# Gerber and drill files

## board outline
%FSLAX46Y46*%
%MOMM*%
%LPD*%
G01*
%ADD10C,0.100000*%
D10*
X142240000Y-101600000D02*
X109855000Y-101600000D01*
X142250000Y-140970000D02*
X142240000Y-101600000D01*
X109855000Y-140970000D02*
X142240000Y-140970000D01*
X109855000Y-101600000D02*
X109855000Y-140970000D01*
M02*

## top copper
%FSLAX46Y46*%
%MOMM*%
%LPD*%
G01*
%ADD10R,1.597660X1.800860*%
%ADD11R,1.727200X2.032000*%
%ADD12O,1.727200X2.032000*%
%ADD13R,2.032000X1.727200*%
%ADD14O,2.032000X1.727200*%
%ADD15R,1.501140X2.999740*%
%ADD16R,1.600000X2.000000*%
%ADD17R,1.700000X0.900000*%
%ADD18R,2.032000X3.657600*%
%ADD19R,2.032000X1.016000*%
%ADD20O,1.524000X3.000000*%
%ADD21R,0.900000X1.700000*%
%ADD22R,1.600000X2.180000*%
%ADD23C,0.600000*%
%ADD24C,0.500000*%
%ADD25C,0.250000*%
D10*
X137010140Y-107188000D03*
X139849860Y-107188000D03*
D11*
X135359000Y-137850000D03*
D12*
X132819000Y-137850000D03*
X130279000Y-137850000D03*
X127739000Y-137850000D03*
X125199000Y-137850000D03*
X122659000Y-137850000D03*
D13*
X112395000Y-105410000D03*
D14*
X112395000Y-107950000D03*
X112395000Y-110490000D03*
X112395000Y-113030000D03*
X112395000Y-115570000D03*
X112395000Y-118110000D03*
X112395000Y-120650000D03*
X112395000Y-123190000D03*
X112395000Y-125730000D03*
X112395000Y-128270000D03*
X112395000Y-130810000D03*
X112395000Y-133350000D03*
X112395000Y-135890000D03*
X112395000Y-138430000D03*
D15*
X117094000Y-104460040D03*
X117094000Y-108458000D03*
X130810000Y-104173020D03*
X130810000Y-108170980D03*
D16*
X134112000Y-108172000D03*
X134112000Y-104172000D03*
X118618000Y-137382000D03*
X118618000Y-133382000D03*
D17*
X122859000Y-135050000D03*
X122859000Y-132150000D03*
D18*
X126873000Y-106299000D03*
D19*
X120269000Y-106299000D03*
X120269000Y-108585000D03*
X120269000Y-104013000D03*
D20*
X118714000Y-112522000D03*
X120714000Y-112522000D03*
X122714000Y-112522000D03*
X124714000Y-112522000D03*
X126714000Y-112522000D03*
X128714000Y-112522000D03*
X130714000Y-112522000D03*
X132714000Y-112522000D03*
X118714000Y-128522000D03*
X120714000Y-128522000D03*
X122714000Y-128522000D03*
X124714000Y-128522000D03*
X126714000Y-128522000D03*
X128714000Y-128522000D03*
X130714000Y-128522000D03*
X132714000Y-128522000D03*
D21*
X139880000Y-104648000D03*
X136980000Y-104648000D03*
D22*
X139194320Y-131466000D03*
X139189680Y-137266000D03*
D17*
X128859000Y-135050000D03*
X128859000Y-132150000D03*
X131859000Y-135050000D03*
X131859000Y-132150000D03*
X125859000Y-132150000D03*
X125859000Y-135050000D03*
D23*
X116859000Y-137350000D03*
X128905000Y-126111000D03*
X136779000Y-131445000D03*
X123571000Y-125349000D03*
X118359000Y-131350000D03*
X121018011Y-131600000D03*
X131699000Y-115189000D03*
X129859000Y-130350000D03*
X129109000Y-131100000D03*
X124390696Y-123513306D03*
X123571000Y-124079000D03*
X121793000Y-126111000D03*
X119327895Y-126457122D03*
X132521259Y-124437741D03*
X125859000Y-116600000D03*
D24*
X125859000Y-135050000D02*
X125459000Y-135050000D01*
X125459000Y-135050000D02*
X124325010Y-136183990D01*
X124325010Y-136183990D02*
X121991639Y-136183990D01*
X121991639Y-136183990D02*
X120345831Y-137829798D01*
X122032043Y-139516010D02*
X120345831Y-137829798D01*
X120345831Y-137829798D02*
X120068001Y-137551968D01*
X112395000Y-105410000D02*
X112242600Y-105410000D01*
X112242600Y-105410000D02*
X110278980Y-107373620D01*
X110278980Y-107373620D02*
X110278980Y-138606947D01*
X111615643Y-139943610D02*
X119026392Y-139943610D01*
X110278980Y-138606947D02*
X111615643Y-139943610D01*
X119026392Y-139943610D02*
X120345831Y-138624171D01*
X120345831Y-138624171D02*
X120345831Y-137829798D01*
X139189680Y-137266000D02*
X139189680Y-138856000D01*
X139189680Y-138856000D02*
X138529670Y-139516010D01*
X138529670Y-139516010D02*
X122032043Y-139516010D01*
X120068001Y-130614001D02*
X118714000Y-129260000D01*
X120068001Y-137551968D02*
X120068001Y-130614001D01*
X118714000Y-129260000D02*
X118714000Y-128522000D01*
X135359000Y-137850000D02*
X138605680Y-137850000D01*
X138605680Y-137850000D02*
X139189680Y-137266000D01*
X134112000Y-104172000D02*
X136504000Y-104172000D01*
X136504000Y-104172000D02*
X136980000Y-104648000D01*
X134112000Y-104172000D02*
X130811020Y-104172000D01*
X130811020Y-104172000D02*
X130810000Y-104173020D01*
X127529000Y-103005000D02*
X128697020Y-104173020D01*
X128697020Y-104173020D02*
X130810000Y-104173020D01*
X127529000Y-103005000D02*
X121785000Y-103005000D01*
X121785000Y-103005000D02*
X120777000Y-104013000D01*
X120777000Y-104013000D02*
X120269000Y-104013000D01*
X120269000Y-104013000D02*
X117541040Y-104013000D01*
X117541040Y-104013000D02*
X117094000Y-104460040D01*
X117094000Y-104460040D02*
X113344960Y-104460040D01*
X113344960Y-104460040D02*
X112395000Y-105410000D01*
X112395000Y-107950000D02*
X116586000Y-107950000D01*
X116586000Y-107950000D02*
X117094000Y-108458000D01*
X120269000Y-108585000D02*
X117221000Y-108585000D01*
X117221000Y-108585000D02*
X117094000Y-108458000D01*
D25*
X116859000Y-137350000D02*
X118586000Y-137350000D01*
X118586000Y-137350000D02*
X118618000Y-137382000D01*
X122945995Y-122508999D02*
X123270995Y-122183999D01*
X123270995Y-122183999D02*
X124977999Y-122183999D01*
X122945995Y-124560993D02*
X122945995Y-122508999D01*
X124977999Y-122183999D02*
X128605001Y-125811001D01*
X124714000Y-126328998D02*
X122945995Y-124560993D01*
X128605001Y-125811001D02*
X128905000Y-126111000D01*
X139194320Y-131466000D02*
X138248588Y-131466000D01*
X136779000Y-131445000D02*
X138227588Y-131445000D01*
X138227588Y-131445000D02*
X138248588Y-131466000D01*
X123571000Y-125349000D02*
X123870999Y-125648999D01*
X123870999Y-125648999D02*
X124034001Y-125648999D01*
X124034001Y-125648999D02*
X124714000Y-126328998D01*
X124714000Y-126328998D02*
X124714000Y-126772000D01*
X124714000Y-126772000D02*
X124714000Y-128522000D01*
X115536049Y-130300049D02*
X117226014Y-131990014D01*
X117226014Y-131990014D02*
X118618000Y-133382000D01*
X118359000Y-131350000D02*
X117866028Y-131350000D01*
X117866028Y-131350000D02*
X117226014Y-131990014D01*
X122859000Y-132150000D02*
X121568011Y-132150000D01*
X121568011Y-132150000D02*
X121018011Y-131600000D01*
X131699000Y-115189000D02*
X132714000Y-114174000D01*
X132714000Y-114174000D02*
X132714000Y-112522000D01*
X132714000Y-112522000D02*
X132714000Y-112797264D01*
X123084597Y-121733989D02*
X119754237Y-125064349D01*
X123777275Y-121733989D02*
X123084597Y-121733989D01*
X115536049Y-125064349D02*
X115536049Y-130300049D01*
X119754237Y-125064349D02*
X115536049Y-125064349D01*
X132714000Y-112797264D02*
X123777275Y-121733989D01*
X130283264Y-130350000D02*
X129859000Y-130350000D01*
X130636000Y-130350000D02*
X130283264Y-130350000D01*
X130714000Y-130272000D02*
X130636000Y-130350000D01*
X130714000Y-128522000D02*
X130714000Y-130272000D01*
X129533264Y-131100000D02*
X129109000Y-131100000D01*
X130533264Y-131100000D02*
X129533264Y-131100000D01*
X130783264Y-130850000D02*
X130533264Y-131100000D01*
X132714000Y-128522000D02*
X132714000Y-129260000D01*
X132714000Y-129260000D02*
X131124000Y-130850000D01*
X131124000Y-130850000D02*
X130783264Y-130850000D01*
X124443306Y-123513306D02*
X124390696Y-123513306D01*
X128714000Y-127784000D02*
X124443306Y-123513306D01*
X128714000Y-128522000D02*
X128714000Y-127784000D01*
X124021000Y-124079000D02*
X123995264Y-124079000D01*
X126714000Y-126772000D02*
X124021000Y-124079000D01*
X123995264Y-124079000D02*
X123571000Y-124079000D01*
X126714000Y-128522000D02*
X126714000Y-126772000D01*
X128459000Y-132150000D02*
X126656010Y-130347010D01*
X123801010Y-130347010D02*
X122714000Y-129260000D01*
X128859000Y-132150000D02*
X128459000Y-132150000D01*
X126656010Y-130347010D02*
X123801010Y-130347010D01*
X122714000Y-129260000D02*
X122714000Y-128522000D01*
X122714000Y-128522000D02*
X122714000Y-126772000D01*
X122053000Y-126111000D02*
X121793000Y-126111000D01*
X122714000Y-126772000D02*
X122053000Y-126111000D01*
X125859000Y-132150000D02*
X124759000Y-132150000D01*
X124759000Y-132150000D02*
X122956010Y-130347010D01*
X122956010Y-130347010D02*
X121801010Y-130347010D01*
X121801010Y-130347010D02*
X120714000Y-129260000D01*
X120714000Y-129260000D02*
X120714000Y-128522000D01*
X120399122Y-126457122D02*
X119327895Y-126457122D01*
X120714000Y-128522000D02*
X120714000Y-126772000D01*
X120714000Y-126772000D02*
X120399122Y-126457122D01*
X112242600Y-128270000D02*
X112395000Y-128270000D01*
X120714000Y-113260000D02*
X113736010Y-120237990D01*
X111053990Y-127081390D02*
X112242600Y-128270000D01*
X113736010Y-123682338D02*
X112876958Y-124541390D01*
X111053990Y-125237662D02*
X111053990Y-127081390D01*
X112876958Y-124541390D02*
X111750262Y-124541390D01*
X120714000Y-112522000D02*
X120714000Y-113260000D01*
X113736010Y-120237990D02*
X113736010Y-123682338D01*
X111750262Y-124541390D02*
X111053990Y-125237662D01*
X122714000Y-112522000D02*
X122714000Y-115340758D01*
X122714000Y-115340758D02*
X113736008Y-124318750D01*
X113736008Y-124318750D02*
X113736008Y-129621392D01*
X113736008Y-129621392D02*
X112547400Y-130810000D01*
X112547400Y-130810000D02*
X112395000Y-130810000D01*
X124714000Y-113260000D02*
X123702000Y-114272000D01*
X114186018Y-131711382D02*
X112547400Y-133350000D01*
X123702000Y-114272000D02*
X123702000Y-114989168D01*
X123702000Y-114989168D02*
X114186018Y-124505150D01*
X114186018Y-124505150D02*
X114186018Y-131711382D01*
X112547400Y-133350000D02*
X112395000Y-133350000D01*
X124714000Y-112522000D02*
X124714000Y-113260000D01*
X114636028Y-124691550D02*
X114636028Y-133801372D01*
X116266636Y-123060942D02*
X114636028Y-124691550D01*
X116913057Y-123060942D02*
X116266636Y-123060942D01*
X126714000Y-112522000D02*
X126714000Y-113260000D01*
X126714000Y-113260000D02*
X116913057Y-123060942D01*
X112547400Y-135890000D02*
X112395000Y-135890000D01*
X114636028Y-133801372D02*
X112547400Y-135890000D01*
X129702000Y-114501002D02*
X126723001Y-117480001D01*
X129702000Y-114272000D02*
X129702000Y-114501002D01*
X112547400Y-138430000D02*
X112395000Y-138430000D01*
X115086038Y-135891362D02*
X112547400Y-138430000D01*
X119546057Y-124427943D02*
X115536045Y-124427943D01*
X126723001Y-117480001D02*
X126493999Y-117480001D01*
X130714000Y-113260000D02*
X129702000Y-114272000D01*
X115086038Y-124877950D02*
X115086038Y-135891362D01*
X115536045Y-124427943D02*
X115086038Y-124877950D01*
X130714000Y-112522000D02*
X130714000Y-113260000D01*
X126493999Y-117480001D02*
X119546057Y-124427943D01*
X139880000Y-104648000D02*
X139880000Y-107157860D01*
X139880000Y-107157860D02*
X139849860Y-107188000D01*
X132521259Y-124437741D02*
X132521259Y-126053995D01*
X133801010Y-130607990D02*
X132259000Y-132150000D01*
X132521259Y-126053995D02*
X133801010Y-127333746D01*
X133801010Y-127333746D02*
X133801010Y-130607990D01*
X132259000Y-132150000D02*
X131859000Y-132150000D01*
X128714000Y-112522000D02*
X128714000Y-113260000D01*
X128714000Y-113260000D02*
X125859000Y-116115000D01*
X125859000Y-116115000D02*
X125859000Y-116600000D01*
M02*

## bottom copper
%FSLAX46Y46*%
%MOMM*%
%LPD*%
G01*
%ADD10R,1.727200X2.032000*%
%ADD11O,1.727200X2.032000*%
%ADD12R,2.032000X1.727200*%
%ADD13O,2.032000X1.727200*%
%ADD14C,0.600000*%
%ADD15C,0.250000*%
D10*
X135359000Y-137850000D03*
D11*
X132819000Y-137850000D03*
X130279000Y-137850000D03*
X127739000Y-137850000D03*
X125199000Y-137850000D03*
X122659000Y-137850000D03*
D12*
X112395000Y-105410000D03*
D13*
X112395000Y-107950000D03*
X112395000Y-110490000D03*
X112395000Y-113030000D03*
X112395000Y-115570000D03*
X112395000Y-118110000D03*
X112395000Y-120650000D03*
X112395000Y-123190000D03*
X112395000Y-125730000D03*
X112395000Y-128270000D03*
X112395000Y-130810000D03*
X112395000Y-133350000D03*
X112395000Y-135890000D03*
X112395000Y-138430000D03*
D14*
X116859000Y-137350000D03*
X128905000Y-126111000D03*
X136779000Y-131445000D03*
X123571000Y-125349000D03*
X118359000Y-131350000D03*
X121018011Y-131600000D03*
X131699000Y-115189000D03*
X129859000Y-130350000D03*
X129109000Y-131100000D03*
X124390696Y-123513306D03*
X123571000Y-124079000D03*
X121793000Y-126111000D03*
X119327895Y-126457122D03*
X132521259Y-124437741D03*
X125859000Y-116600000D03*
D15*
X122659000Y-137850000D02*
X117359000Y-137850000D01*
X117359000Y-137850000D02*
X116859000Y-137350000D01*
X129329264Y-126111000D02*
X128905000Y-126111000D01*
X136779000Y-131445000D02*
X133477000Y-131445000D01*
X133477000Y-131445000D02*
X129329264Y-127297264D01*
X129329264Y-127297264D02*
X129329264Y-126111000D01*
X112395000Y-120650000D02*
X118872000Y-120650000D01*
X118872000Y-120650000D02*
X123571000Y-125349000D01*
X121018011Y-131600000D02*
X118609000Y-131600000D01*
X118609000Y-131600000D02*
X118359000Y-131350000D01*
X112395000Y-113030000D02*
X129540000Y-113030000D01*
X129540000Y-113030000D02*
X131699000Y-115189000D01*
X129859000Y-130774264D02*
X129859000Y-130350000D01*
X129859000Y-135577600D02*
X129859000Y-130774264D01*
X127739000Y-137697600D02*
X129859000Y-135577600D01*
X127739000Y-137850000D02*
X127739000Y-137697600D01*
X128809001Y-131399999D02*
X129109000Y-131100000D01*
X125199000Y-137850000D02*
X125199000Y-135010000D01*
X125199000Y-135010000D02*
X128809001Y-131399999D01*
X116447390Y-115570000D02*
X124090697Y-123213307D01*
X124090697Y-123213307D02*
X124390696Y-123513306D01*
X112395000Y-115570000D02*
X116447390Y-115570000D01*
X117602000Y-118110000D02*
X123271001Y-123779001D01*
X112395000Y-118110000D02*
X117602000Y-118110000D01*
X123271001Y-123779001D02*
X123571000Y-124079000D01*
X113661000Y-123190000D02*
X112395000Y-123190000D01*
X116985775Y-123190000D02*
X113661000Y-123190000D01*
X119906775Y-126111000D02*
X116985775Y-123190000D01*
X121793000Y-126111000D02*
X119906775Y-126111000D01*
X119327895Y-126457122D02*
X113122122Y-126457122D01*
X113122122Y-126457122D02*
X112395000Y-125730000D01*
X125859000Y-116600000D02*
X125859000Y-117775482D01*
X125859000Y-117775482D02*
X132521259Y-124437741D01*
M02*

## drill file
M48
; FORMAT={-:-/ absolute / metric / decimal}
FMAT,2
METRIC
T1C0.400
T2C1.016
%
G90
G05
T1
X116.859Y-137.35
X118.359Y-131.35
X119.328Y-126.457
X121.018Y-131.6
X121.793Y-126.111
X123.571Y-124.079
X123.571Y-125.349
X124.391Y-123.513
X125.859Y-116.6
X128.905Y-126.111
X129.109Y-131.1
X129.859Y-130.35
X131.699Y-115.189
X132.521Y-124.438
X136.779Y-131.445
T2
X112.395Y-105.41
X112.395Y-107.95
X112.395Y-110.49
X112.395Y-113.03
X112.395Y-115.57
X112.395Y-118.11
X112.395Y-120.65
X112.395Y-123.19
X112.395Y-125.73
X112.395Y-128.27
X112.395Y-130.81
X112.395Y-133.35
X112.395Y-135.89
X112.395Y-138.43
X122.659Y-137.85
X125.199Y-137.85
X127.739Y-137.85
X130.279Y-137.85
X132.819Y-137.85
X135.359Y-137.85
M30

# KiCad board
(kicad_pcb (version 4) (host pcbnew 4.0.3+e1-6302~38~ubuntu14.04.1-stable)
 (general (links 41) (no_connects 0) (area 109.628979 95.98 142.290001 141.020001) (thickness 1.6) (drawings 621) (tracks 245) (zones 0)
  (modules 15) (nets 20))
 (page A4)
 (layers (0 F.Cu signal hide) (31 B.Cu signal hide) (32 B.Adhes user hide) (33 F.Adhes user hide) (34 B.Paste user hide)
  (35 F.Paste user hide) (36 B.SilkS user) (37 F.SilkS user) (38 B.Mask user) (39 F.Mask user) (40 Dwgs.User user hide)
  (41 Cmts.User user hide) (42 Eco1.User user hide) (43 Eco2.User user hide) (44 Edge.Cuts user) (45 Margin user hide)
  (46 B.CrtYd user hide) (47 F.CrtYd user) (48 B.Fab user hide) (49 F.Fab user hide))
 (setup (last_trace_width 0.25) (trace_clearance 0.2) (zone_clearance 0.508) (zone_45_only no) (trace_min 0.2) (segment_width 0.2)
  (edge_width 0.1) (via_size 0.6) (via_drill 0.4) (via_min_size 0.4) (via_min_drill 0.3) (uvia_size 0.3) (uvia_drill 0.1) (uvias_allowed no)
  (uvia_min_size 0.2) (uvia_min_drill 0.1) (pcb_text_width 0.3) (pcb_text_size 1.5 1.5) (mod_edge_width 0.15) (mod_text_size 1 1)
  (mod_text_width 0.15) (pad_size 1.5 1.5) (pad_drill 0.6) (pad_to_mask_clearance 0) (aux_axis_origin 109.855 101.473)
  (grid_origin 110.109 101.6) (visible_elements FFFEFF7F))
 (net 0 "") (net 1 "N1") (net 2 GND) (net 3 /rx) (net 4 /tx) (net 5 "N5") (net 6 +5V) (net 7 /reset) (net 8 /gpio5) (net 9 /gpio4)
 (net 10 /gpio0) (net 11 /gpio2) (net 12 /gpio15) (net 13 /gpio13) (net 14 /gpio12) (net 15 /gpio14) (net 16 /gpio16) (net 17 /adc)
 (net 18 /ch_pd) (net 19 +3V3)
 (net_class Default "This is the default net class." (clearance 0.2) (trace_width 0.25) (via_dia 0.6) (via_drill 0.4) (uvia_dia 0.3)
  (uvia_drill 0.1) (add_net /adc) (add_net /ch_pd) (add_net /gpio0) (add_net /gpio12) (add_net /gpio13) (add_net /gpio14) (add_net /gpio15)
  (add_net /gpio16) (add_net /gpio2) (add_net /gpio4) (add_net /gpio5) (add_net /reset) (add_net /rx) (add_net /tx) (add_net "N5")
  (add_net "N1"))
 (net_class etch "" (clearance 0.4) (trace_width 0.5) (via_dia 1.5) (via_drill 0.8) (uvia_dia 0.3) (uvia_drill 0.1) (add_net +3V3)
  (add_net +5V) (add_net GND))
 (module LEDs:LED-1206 (layer F.Cu) (at 138.43 107.188 180)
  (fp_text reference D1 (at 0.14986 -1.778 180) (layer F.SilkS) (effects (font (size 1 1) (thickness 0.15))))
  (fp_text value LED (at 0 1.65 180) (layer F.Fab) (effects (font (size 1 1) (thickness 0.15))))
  (pad 2 smd rect (at 1.41986 0) (size 1.59766 1.80086) (layers F.Cu F.Paste F.Mask))
  (pad 1 smd rect (at -1.41986 0) (size 1.59766 1.80086) (layers F.Cu F.Paste F.Mask) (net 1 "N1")))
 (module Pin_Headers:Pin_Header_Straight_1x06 (layer F.Cu) (at 135.359 137.85 270)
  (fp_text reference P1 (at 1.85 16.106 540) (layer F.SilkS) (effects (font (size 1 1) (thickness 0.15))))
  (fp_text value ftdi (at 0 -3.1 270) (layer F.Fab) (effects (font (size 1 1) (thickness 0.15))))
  (pad 1 thru_hole rect (at 0 0 270) (size 2.032 1.7272) (drill 1.016) (layers *.Cu *.Mask F.SilkS) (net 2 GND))
  (pad 2 thru_hole oval (at 0 2.54 270) (size 2.032 1.7272) (drill 1.016) (layers *.Cu *.Mask F.SilkS))
  (pad 3 thru_hole oval (at 0 5.08 270) (size 2.032 1.7272) (drill 1.016) (layers *.Cu *.Mask F.SilkS))
  (pad 4 thru_hole oval (at 0 7.62 270) (size 2.032 1.7272) (drill 1.016) (layers *.Cu *.Mask F.SilkS) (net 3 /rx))
  (pad 5 thru_hole oval (at 0 10.16 270) (size 2.032 1.7272) (drill 1.016) (layers *.Cu *.Mask F.SilkS) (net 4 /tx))
  (pad 6 thru_hole oval (at 0 12.7 270) (size 2.032 1.7272) (drill 1.016) (layers *.Cu *.Mask F.SilkS) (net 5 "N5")))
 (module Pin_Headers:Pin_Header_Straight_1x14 (layer B.Cu) (at 112.395 105.41 180)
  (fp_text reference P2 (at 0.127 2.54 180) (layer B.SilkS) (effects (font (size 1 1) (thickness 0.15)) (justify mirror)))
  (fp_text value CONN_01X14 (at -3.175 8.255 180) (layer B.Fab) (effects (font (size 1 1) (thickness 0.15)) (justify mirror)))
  (pad 1 thru_hole rect (at 0 0 180) (size 2.032 1.7272) (drill 1.016) (layers *.Cu *.Mask B.SilkS) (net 2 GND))
  (pad 2 thru_hole oval (at 0 -2.54 180) (size 2.032 1.7272) (drill 1.016) (layers *.Cu *.Mask B.SilkS) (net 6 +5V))
  (pad 3 thru_hole oval (at 0 -5.08 180) (size 2.032 1.7272) (drill 1.016) (layers *.Cu *.Mask B.SilkS))
  (pad 4 thru_hole oval (at 0 -7.62 180) (size 2.032 1.7272) (drill 1.016) (layers *.Cu *.Mask B.SilkS) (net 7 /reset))
  (pad 5 thru_hole oval (at 0 -10.16 180) (size 2.032 1.7272) (drill 1.016) (layers *.Cu *.Mask B.SilkS) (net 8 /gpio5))
  (pad 6 thru_hole oval (at 0 -12.7 180) (size 2.032 1.7272) (drill 1.016) (layers *.Cu *.Mask B.SilkS) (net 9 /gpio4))
  (pad 7 thru_hole oval (at 0 -15.24 180) (size 2.032 1.7272) (drill 1.016) (layers *.Cu *.Mask B.SilkS) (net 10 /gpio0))
  (pad 8 thru_hole oval (at 0 -17.78 180) (size 2.032 1.7272) (drill 1.016) (layers *.Cu *.Mask B.SilkS) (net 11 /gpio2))
  (pad 9 thru_hole oval (at 0 -20.32 180) (size 2.032 1.7272) (drill 1.016) (layers *.Cu *.Mask B.SilkS) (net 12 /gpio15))
  (pad 10 thru_hole oval (at 0 -22.86 180) (size 2.032 1.7272) (drill 1.016) (layers *.Cu *.Mask B.SilkS) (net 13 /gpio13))
  (pad 11 thru_hole oval (at 0 -25.4 180) (size 2.032 1.7272) (drill 1.016) (layers *.Cu *.Mask B.SilkS) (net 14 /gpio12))
  (pad 12 thru_hole oval (at 0 -27.94 180) (size 2.032 1.7272) (drill 1.016) (layers *.Cu *.Mask B.SilkS) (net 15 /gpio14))
  (pad 13 thru_hole oval (at 0 -30.48 180) (size 2.032 1.7272) (drill 1.016) (layers *.Cu *.Mask B.SilkS) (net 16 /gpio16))
  (pad 14 thru_hole oval (at 0 -33.02 180) (size 2.032 1.7272) (drill 1.016) (layers *.Cu *.Mask B.SilkS) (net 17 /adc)))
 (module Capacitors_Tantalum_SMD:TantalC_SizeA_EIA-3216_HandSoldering (layer F.Cu) (at 117.094 106.45902 90)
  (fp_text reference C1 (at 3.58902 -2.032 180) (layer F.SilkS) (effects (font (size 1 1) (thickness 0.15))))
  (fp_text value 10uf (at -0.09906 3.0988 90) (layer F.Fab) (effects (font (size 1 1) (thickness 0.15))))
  (pad 2 smd rect (at 1.99898 0 90) (size 2.99974 1.50114) (layers F.Cu F.Paste F.Mask) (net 2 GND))
  (pad 1 smd rect (at -1.99898 0 90) (size 2.99974 1.50114) (layers F.Cu F.Paste F.Mask) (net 6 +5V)))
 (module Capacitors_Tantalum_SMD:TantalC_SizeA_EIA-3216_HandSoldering (layer F.Cu) (at 130.81 106.172 90)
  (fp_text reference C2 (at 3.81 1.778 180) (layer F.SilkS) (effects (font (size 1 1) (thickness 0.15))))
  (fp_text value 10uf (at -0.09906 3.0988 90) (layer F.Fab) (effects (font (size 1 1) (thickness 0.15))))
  (pad 2 smd rect (at 1.99898 0 90) (size 2.99974 1.50114) (layers F.Cu F.Paste F.Mask) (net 2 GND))
  (pad 1 smd rect (at -1.99898 0 90) (size 2.99974 1.50114) (layers F.Cu F.Paste F.Mask)))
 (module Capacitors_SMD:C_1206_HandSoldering (layer F.Cu) (at 134.112 106.172 90)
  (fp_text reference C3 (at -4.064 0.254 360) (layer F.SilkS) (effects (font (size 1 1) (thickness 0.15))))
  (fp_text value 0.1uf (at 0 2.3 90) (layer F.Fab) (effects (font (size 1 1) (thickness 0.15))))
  (pad 1 smd rect (at -2 0 90) (size 2 1.6) (layers F.Cu F.Paste F.Mask))
  (pad 2 smd rect (at 2 0 90) (size 2 1.6) (layers F.Cu F.Paste F.Mask) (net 2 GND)))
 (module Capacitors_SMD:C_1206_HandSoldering (layer F.Cu) (at 118.618 135.382 90)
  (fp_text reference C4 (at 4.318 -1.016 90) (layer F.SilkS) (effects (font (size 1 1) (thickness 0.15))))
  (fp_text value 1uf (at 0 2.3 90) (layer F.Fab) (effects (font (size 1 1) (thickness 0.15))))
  (pad 1 smd rect (at -2 0 90) (size 2 1.6) (layers F.Cu F.Paste F.Mask) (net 5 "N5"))
  (pad 2 smd rect (at 2 0 90) (size 2 1.6) (layers F.Cu F.Paste F.Mask) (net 7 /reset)))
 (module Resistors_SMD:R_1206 (layer F.Cu) (at 122.859 133.6 90)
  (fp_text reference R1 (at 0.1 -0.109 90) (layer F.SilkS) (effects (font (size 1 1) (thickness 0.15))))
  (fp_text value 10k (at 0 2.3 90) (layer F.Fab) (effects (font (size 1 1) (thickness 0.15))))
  (pad 1 smd rect (at -1.45 0 90) (size 0.9 1.7) (layers F.Cu F.Paste F.Mask))
  (pad 2 smd rect (at 1.45 0 90) (size 0.9 1.7) (layers F.Cu F.Paste F.Mask) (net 7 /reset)))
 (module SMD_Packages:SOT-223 (layer F.Cu) (at 123.571 106.299 270)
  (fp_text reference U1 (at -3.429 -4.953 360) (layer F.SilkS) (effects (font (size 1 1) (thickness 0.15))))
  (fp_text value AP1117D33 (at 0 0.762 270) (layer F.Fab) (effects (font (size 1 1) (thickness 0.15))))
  (pad 4 smd rect (at 0 -3.302 270) (size 3.6576 2.032) (layers F.Cu F.Paste F.Mask))
  (pad 2 smd rect (at 0 3.302 270) (size 1.016 2.032) (layers F.Cu F.Paste F.Mask))
  (pad 3 smd rect (at 2.286 3.302 270) (size 1.016 2.032) (layers F.Cu F.Paste F.Mask) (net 6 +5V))
  (pad 1 smd rect (at -2.286 3.302 270) (size 1.016 2.032) (layers F.Cu F.Paste F.Mask) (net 2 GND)))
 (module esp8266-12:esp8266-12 (layer F.Cu) (at 118.714 112.622)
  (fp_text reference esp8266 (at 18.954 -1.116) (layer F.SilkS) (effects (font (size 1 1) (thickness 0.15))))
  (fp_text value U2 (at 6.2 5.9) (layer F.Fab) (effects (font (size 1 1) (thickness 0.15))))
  (pad 8 smd oval (at 0 -0.1) (size 1.524 3) (layers F.Cu F.Paste F.Mask))
  (pad 7 smd oval (at 2 -0.1) (size 1.524 3) (layers F.Cu F.Paste F.Mask) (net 13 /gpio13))
  (pad 6 smd oval (at 4 -0.1) (size 1.524 3) (layers F.Cu F.Paste F.Mask) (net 14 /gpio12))
  (pad 5 smd oval (at 6 -0.1) (size 1.524 3) (layers F.Cu F.Paste F.Mask) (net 15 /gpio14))
  (pad 4 smd oval (at 8 -0.1) (size 1.524 3) (layers F.Cu F.Paste F.Mask) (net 16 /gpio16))
  (pad 3 smd oval (at 10 -0.1) (size 1.524 3) (layers F.Cu F.Paste F.Mask) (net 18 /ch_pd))
  (pad 2 smd oval (at 12 -0.1) (size 1.524 3) (layers F.Cu F.Paste F.Mask) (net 17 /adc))
  (pad 1 smd oval (at 14 -0.1) (size 1.524 3) (layers F.Cu F.Paste F.Mask) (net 7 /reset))
  (pad 9 smd oval (at 0 15.9) (size 1.524 3) (layers F.Cu F.Paste F.Mask) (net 2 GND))
  (pad 10 smd oval (at 2 15.9) (size 1.524 3) (layers F.Cu F.Paste F.Mask) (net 12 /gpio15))
  (pad 11 smd oval (at 4 15.9) (size 1.524 3) (layers F.Cu F.Paste F.Mask) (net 11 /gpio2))
  (pad 12 smd oval (at 6 15.9) (size 1.524 3) (layers F.Cu F.Paste F.Mask) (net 10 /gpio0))
  (pad 13 smd oval (at 8 15.9) (size 1.524 3) (layers F.Cu F.Paste F.Mask) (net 9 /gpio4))
  (pad 14 smd oval (at 10 15.9) (size 1.524 3) (layers F.Cu F.Paste F.Mask) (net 8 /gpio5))
  (pad 15 smd oval (at 12 15.9) (size 1.524 3) (layers F.Cu F.Paste F.Mask) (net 3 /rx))
  (pad 16 smd oval (at 14 15.9) (size 1.524 3) (layers F.Cu F.Paste F.Mask) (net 4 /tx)))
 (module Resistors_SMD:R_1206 (layer F.Cu) (at 138.43 104.648 180)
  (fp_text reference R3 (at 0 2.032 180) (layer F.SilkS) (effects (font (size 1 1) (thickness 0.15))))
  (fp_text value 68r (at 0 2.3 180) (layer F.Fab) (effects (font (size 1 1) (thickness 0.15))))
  (pad 1 smd rect (at -1.45 0 180) (size 0.9 1.7) (layers F.Cu F.Paste F.Mask) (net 1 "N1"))
  (pad 2 smd rect (at 1.45 0 180) (size 0.9 1.7) (layers F.Cu F.Paste F.Mask) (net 2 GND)))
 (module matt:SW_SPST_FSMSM (layer F.Cu) (at 139.192 134.366 270)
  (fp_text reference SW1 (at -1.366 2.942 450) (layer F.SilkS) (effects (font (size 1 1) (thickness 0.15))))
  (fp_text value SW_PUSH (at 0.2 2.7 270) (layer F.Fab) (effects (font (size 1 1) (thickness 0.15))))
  (pad 1 smd rect (at -2.9 -0.00232 270) (size 2.18 1.6) (layers F.Cu F.Paste F.Mask) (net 10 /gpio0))
  (pad 2 smd rect (at 2.9 0.00232 270) (size 2.18 1.6) (layers F.Cu F.Paste F.Mask) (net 2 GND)))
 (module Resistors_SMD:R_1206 (layer F.Cu) (at 128.859 133.6 90)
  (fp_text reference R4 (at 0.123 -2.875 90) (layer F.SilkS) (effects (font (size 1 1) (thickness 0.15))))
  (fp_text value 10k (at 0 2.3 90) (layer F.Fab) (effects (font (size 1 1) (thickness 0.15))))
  (pad 1 smd rect (at -1.45 0 90) (size 0.9 1.7) (layers F.Cu F.Paste F.Mask))
  (pad 2 smd rect (at 1.45 0 90) (size 0.9 1.7) (layers F.Cu F.Paste F.Mask) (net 11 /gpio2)))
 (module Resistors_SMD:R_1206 (layer F.Cu) (at 131.859 133.6 90)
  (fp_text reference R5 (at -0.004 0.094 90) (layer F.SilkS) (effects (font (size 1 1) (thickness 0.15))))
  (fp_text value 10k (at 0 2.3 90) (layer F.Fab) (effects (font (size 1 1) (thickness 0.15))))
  (pad 1 smd rect (at -1.45 0 90) (size 0.9 1.7) (layers F.Cu F.Paste F.Mask))
  (pad 2 smd rect (at 1.45 0 90) (size 0.9 1.7) (layers F.Cu F.Paste F.Mask) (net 18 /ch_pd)))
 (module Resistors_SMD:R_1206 (layer F.Cu) (at 125.859 133.6 270)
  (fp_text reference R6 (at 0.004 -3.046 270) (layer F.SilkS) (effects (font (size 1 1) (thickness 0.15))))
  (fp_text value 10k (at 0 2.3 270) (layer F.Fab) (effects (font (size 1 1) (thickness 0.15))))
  (pad 1 smd rect (at -1.45 0 270) (size 0.9 1.7) (layers F.Cu F.Paste F.Mask) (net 12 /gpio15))
  (pad 2 smd rect (at 1.45 0 270) (size 0.9 1.7) (layers F.Cu F.Paste F.Mask) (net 2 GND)))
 (gr_line (start 142.24 101.6) (end 109.855 101.6) (layer Edge.Cuts) (width 0.1))
 (gr_line (start 142.25 140.97) (end 142.24 101.6) (layer Edge.Cuts) (width 0.1))
 (gr_line (start 109.855 140.97) (end 142.24 140.97) (layer Edge.Cuts) (width 0.1))
 (gr_line (start 109.855 101.6) (end 109.855 140.97) (layer Edge.Cuts) (width 0.1))
 (segment (start 125.859 135.05) (end 125.459 135.05) (width 0.5) (layer F.Cu) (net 2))
 (segment (start 125.459 135.05) (end 124.32501 136.18399) (width 0.5) (layer F.Cu) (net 2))
 (segment (start 124.32501 136.18399) (end 121.991639 136.18399) (width 0.5) (layer F.Cu) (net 2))
 (segment (start 121.991639 136.18399) (end 120.345831 137.829798) (width 0.5) (layer F.Cu) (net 2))
 (segment (start 122.032043 139.51601) (end 120.345831 137.829798) (width 0.5) (layer F.Cu) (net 2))
 (segment (start 120.345831 137.829798) (end 120.068001 137.551968) (width 0.5) (layer F.Cu) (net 2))
 (segment (start 112.395 105.41) (end 112.2426 105.41) (width 0.5) (layer F.Cu) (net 2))
 (segment (start 112.2426 105.41) (end 110.27898 107.37362) (width 0.5) (layer F.Cu) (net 2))
 (segment (start 110.27898 107.37362) (end 110.27898 138.606947) (width 0.5) (layer F.Cu) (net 2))
 (segment (start 111.615643 139.94361) (end 119.026392 139.94361) (width 0.5) (layer F.Cu) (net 2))
 (segment (start 110.27898 138.606947) (end 111.615643 139.94361) (width 0.5) (layer F.Cu) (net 2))
 (segment (start 119.026392 139.94361) (end 120.345831 138.624171) (width 0.5) (layer F.Cu) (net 2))
 (segment (start 120.345831 138.624171) (end 120.345831 137.829798) (width 0.5) (layer F.Cu) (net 2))
 (segment (start 139.18968 137.266) (end 139.18968 138.856) (width 0.5) (layer F.Cu) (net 2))
 (segment (start 139.18968 138.856) (end 138.52967 139.51601) (width 0.5) (layer F.Cu) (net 2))
 (segment (start 138.52967 139.51601) (end 122.032043 139.51601) (width 0.5) (layer F.Cu) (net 2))
 (segment (start 120.068001 130.614001) (end 118.714 129.26) (width 0.5) (layer F.Cu) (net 2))
 (segment (start 120.068001 137.551968) (end 120.068001 130.614001) (width 0.5) (layer F.Cu) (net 2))
 (segment (start 118.714 129.26) (end 118.714 128.522) (width 0.5) (layer F.Cu) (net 2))
 (segment (start 135.359 137.85) (end 138.60568 137.85) (width 0.5) (layer F.Cu) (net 2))
 (segment (start 138.60568 137.85) (end 139.18968 137.266) (width 0.5) (layer F.Cu) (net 2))
 (segment (start 134.112 104.172) (end 136.504 104.172) (width 0.5) (layer F.Cu) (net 2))
 (segment (start 136.504 104.172) (end 136.98 104.648) (width 0.5) (layer F.Cu) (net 2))
 (segment (start 134.112 104.172) (end 130.81102 104.172) (width 0.5) (layer F.Cu) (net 2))
 (segment (start 130.81102 104.172) (end 130.81 104.17302) (width 0.5) (layer F.Cu) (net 2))
 (segment (start 127.529 103.005) (end 128.69702 104.17302) (width 0.5) (layer F.Cu) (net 2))
 (segment (start 128.69702 104.17302) (end 130.81 104.17302) (width 0.5) (layer F.Cu) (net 2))
 (segment (start 127.529 103.005) (end 121.785 103.005) (width 0.5) (layer F.Cu) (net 2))
 (segment (start 121.785 103.005) (end 120.777 104.013) (width 0.5) (layer F.Cu) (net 2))
 (segment (start 120.777 104.013) (end 120.269 104.013) (width 0.5) (layer F.Cu) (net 2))
 (segment (start 120.269 104.013) (end 117.54104 104.013) (width 0.5) (layer F.Cu) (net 2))
 (segment (start 117.54104 104.013) (end 117.094 104.46004) (width 0.5) (layer F.Cu) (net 2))
 (segment (start 117.094 104.46004) (end 113.34496 104.46004) (width 0.5) (layer F.Cu) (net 2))
 (segment (start 113.34496 104.46004) (end 112.395 105.41) (width 0.5) (layer F.Cu) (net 2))
 (segment (start 112.395 107.95) (end 116.586 107.95) (width 0.5) (layer F.Cu) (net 6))
 (segment (start 116.586 107.95) (end 117.094 108.458) (width 0.5) (layer F.Cu) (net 6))
 (segment (start 120.269 108.585) (end 117.221 108.585) (width 0.5) (layer F.Cu) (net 6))
 (segment (start 117.221 108.585) (end 117.094 108.458) (width 0.5) (layer F.Cu) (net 6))
 (segment (start 116.859 137.35) (end 118.586 137.35) (width 0.25) (layer F.Cu) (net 5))
 (segment (start 118.586 137.35) (end 118.618 137.382) (width 0.25) (layer F.Cu) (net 5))
 (segment (start 122.659 137.85) (end 117.359 137.85) (width 0.25) (layer B.Cu) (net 5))
 (segment (start 117.359 137.85) (end 116.859 137.35) (width 0.25) (layer B.Cu) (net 5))
 (segment (start 122.945995 122.508999) (end 123.270995 122.183999) (width 0.25) (layer F.Cu) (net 10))
 (segment (start 123.270995 122.183999) (end 124.977999 122.183999) (width 0.25) (layer F.Cu) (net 10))
 (segment (start 122.945995 124.560993) (end 122.945995 122.508999) (width 0.25) (layer F.Cu) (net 10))
 (segment (start 124.977999 122.183999) (end 128.605001 125.811001) (width 0.25) (layer F.Cu) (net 10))
 (segment (start 124.714 126.328998) (end 122.945995 124.560993) (width 0.25) (layer F.Cu) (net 10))
 (segment (start 128.605001 125.811001) (end 128.905 126.111) (width 0.25) (layer F.Cu) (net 10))
 (segment (start 129.329264 126.111) (end 128.905 126.111) (width 0.25) (layer B.Cu) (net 10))
 (segment (start 136.779 131.445) (end 133.477 131.445) (width 0.25) (layer B.Cu) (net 10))
 (segment (start 133.477 131.445) (end 129.329264 127.297264) (width 0.25) (layer B.Cu) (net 10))
 (segment (start 129.329264 127.297264) (end 129.329264 126.111) (width 0.25) (layer B.Cu) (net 10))
 (segment (start 139.19432 131.466) (end 138.248588 131.466) (width 0.25) (layer F.Cu) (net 10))
 (segment (start 136.779 131.445) (end 138.227588 131.445) (width 0.25) (layer F.Cu) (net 10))
 (segment (start 138.227588 131.445) (end 138.248588 131.466) (width 0.25) (layer F.Cu) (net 10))
 (segment (start 123.571 125.349) (end 123.870999 125.648999) (width 0.25) (layer F.Cu) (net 10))
 (segment (start 123.870999 125.648999) (end 124.034001 125.648999) (width 0.25) (layer F.Cu) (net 10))
 (segment (start 124.034001 125.648999) (end 124.714 126.328998) (width 0.25) (layer F.Cu) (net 10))
 (segment (start 112.395 120.65) (end 118.872 120.65) (width 0.25) (layer B.Cu) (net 10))
 (segment (start 118.872 120.65) (end 123.571 125.349) (width 0.25) (layer B.Cu) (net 10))
 (segment (start 124.714 126.328998) (end 124.714 126.772) (width 0.25) (layer F.Cu) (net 10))
 (segment (start 124.714 126.772) (end 124.714 128.522) (width 0.25) (layer F.Cu) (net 10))
 (segment (start 115.536049 130.300049) (end 117.226014 131.990014) (width 0.25) (layer F.Cu) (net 7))
 (segment (start 117.226014 131.990014) (end 118.618 133.382) (width 0.25) (layer F.Cu) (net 7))
 (segment (start 118.359 131.35) (end 117.866028 131.35) (width 0.25) (layer F.Cu) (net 7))
 (segment (start 117.866028 131.35) (end 117.226014 131.990014) (width 0.25) (layer F.Cu) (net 7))
 (segment (start 121.018011 131.6) (end 118.609 131.6) (width 0.25) (layer B.Cu) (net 7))
 (segment (start 118.609 131.6) (end 118.359 131.35) (width 0.25) (layer B.Cu) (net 7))
 (segment (start 122.859 132.15) (end 121.568011 132.15) (width 0.25) (layer F.Cu) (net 7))
 (segment (start 121.568011 132.15) (end 121.018011 131.6) (width 0.25) (layer F.Cu) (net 7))
 (segment (start 131.699 115.189) (end 132.714 114.174) (width 0.25) (layer F.Cu) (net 7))
 (segment (start 132.714 114.174) (end 132.714 112.522) (width 0.25) (layer F.Cu) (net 7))
 (segment (start 112.395 113.03) (end 129.54 113.03) (width 0.25) (layer B.Cu) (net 7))
 (segment (start 129.54 113.03) (end 131.699 115.189) (width 0.25) (layer B.Cu) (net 7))
 (segment (start 132.714 112.522) (end 132.714 112.797264) (width 0.25) (layer F.Cu) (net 7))
 (segment (start 123.084597 121.733989) (end 119.754237 125.064349) (width 0.25) (layer F.Cu) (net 7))
 (segment (start 123.777275 121.733989) (end 123.084597 121.733989) (width 0.25) (layer F.Cu) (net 7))
 (segment (start 115.536049 125.064349) (end 115.536049 130.300049) (width 0.25) (layer F.Cu) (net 7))
 (segment (start 119.754237 125.064349) (end 115.536049 125.064349) (width 0.25) (layer F.Cu) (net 7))
 (segment (start 132.714 112.797264) (end 123.777275 121.733989) (width 0.25) (layer F.Cu) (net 7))
 (segment (start 129.859 130.774264) (end 129.859 130.35) (width 0.25) (layer B.Cu) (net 3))
 (segment (start 129.859 135.5776) (end 129.859 130.774264) (width 0.25) (layer B.Cu) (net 3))
 (segment (start 127.739 137.6976) (end 129.859 135.5776) (width 0.25) (layer B.Cu) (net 3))
 (segment (start 130.283264 130.35) (end 129.859 130.35) (width 0.25) (layer F.Cu) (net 3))
 (segment (start 130.636 130.35) (end 130.283264 130.35) (width 0.25) (layer F.Cu) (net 3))
 (segment (start 127.739 137.85) (end 127.739 137.6976) (width 0.25) (layer B.Cu) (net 3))
 (segment (start 130.714 130.272) (end 130.636 130.35) (width 0.25) (layer F.Cu) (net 3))
 (segment (start 130.714 128.522) (end 130.714 130.272) (width 0.25) (layer F.Cu) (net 3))
 (segment (start 128.809001 131.399999) (end 129.109 131.1) (width 0.25) (layer B.Cu) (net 4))
 (segment (start 125.199 137.85) (end 125.199 135.01) (width 0.25) (layer B.Cu) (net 4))
 (segment (start 125.199 135.01) (end 128.809001 131.399999) (width 0.25) (layer B.Cu) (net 4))
 (segment (start 129.533264 131.1) (end 129.109 131.1) (width 0.25) (layer F.Cu) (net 4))
 (segment (start 130.533264 131.1) (end 129.533264 131.1) (width 0.25) (layer F.Cu) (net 4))
 (segment (start 130.783264 130.85) (end 130.533264 131.1) (width 0.25) (layer F.Cu) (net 4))
 (segment (start 132.714 128.522) (end 132.714 129.26) (width 0.25) (layer F.Cu) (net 4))
 (segment (start 132.714 129.26) (end 131.124 130.85) (width 0.25) (layer F.Cu) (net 4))
 (segment (start 131.124 130.85) (end 130.783264 130.85) (width 0.25) (layer F.Cu) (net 4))
 (segment (start 124.443306 123.513306) (end 124.390696 123.513306) (width 0.25) (layer F.Cu) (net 8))
 (segment (start 128.714 127.784) (end 124.443306 123.513306) (width 0.25) (layer F.Cu) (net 8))
 (segment (start 116.44739 115.57) (end 124.090697 123.213307) (width 0.25) (layer B.Cu) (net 8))
 (segment (start 128.714 128.522) (end 128.714 127.784) (width 0.25) (layer F.Cu) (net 8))
 (segment (start 124.090697 123.213307) (end 124.390696 123.513306) (width 0.25) (layer B.Cu) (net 8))
 (segment (start 112.395 115.57) (end 116.44739 115.57) (width 0.25) (layer B.Cu) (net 8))
 (segment (start 117.602 118.11) (end 123.271001 123.779001) (width 0.25) (layer B.Cu) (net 9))
 (segment (start 112.395 118.11) (end 117.602 118.11) (width 0.25) (layer B.Cu) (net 9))
 (segment (start 124.021 124.079) (end 123.995264 124.079) (width 0.25) (layer F.Cu) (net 9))
 (segment (start 126.714 126.772) (end 124.021 124.079) (width 0.25) (layer F.Cu) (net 9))
 (segment (start 123.995264 124.079) (end 123.571 124.079) (width 0.25) (layer F.Cu) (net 9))
 (segment (start 123.271001 123.779001) (end 123.571 124.079) (width 0.25) (layer B.Cu) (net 9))
 (segment (start 126.714 128.522) (end 126.714 126.772) (width 0.25) (layer F.Cu) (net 9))
 (segment (start 128.459 132.15) (end 126.65601 130.34701) (width 0.25) (layer F.Cu) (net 11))
 (segment (start 123.80101 130.34701) (end 122.714 129.26) (width 0.25) (layer F.Cu) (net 11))
 (segment (start 128.859 132.15) (end 128.459 132.15) (width 0.25) (layer F.Cu) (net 11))
 (segment (start 126.65601 130.34701) (end 123.80101 130.34701) (width 0.25) (layer F.Cu) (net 11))
 (segment (start 122.714 129.26) (end 122.714 128.522) (width 0.25) (layer F.Cu) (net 11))
 (segment (start 113.661 123.19) (end 112.395 123.19) (width 0.25) (layer B.Cu) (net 11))
 (segment (start 116.985775 123.19) (end 113.661 123.19) (width 0.25) (layer B.Cu) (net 11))
 (segment (start 119.906775 126.111) (end 116.985775 123.19) (width 0.25) (layer B.Cu) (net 11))
 (segment (start 121.793 126.111) (end 119.906775 126.111) (width 0.25) (layer B.Cu) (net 11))
 (segment (start 122.714 128.522) (end 122.714 126.772) (width 0.25) (layer F.Cu) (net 11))
 (segment (start 122.053 126.111) (end 121.793 126.111) (width 0.25) (layer F.Cu) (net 11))
 (segment (start 122.714 126.772) (end 122.053 126.111) (width 0.25) (layer F.Cu) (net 11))
 (segment (start 125.859 132.15) (end 124.759 132.15) (width 0.25) (layer F.Cu) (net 12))
 (segment (start 124.759 132.15) (end 122.95601 130.34701) (width 0.25) (layer F.Cu) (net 12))
 (segment (start 122.95601 130.34701) (end 121.80101 130.34701) (width 0.25) (layer F.Cu) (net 12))
 (segment (start 121.80101 130.34701) (end 120.714 129.26) (width 0.25) (layer F.Cu) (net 12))
 (segment (start 120.714 129.26) (end 120.714 128.522) (width 0.25) (layer F.Cu) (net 12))
 (segment (start 119.327895 126.457122) (end 113.122122 126.457122) (width 0.25) (layer B.Cu) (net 12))
 (segment (start 113.122122 126.457122) (end 112.395 125.73) (width 0.25) (layer B.Cu) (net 12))
 (segment (start 120.399122 126.457122) (end 119.327895 126.457122) (width 0.25) (layer F.Cu) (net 12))
 (segment (start 120.714 128.522) (end 120.714 126.772) (width 0.25) (layer F.Cu) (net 12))
 (segment (start 120.714 126.772) (end 120.399122 126.457122) (width 0.25) (layer F.Cu) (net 12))
 (segment (start 112.2426 128.27) (end 112.395 128.27) (width 0.25) (layer F.Cu) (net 13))
 (segment (start 120.714 113.26) (end 113.73601 120.23799) (width 0.25) (layer F.Cu) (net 13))
 (segment (start 111.05399 127.08139) (end 112.2426 128.27) (width 0.25) (layer F.Cu) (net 13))
 (segment (start 113.73601 123.682338) (end 112.876958 124.54139) (width 0.25) (layer F.Cu) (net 13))
 (segment (start 111.05399 125.237662) (end 111.05399 127.08139) (width 0.25) (layer F.Cu) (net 13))
 (segment (start 112.876958 124.54139) (end 111.750262 124.54139) (width 0.25) (layer F.Cu) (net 13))
 (segment (start 120.714 112.522) (end 120.714 113.26) (width 0.25) (layer F.Cu) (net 13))
 (segment (start 113.73601 120.23799) (end 113.73601 123.682338) (width 0.25) (layer F.Cu) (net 13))
 (segment (start 111.750262 124.54139) (end 111.05399 125.237662) (width 0.25) (layer F.Cu) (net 13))
 (segment (start 122.714 112.522) (end 122.714 115.340758) (width 0.25) (layer F.Cu) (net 14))
 (segment (start 122.714 115.340758) (end 113.736008 124.31875) (width 0.25) (layer F.Cu) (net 14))
 (segment (start 113.736008 124.31875) (end 113.736008 129.621392) (width 0.25) (layer F.Cu) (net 14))
 (segment (start 113.736008 129.621392) (end 112.5474 130.81) (width 0.25) (layer F.Cu) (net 14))
 (segment (start 112.5474 130.81) (end 112.395 130.81) (width 0.25) (layer F.Cu) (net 14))
 (segment (start 124.714 113.26) (end 123.702 114.272) (width 0.25) (layer F.Cu) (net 15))
 (segment (start 114.186018 131.711382) (end 112.5474 133.35) (width 0.25) (layer F.Cu) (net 15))
 (segment (start 123.702 114.272) (end 123.702 114.989168) (width 0.25) (layer F.Cu) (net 15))
 (segment (start 123.702 114.989168) (end 114.186018 124.50515) (width 0.25) (layer F.Cu) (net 15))
 (segment (start 114.186018 124.50515) (end 114.186018 131.711382) (width 0.25) (layer F.Cu) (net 15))
 (segment (start 112.5474 133.35) (end 112.395 133.35) (width 0.25) (layer F.Cu) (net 15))
 (segment (start 124.714 112.522) (end 124.714 113.26) (width 0.25) (layer F.Cu) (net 15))
 (segment (start 114.636028 124.69155) (end 114.636028 133.801372) (width 0.25) (layer F.Cu) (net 16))
 (segment (start 116.266636 123.060942) (end 114.636028 124.69155) (width 0.25) (layer F.Cu) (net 16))
 (segment (start 116.913057 123.060942) (end 116.266636 123.060942) (width 0.25) (layer F.Cu) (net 16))
 (segment (start 126.714 112.522) (end 126.714 113.26) (width 0.25) (layer F.Cu) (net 16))
 (segment (start 126.714 113.26) (end 116.913057 123.060942) (width 0.25) (layer F.Cu) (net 16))
 (segment (start 112.5474 135.89) (end 112.395 135.89) (width 0.25) (layer F.Cu) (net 16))
 (segment (start 114.636028 133.801372) (end 112.5474 135.89) (width 0.25) (layer F.Cu) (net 16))
 (segment (start 129.702 114.501002) (end 126.723001 117.480001) (width 0.25) (layer F.Cu) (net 17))
 (segment (start 129.702 114.272) (end 129.702 114.501002) (width 0.25) (layer F.Cu) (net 17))
 (segment (start 112.5474 138.43) (end 112.395 138.43) (width 0.25) (layer F.Cu) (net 17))
 (segment (start 115.086038 135.891362) (end 112.5474 138.43) (width 0.25) (layer F.Cu) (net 17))
 (segment (start 119.546057 124.427943) (end 115.536045 124.427943) (width 0.25) (layer F.Cu) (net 17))
 (segment (start 126.723001 117.480001) (end 126.493999 117.480001) (width 0.25) (layer F.Cu) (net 17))
 (segment (start 130.714 113.26) (end 129.702 114.272) (width 0.25) (layer F.Cu) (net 17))
 (segment (start 115.086038 124.87795) (end 115.086038 135.891362) (width 0.25) (layer F.Cu) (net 17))
 (segment (start 115.536045 124.427943) (end 115.086038 124.87795) (width 0.25) (layer F.Cu) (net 17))
 (segment (start 130.714 112.522) (end 130.714 113.26) (width 0.25) (layer F.Cu) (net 17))
 (segment (start 126.493999 117.480001) (end 119.546057 124.427943) (width 0.25) (layer F.Cu) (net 17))
 (segment (start 139.88 104.648) (end 139.88 107.15786) (width 0.25) (layer F.Cu) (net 1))
 (segment (start 139.88 107.15786) (end 139.84986 107.188) (width 0.25) (layer F.Cu) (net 1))
 (segment (start 132.521259 124.437741) (end 132.521259 126.053995) (width 0.25) (layer F.Cu) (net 18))
 (segment (start 133.80101 130.60799) (end 132.259 132.15) (width 0.25) (layer F.Cu) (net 18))
 (segment (start 132.521259 126.053995) (end 133.80101 127.333746) (width 0.25) (layer F.Cu) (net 18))
 (segment (start 133.80101 127.333746) (end 133.80101 130.60799) (width 0.25) (layer F.Cu) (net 18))
 (segment (start 132.259 132.15) (end 131.859 132.15) (width 0.25) (layer F.Cu) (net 18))
 (segment (start 125.859 116.6) (end 125.859 117.775482) (width 0.25) (layer B.Cu) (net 18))
 (segment (start 125.859 117.775482) (end 132.521259 124.437741) (width 0.25) (layer B.Cu) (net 18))
 (segment (start 128.714 112.522) (end 128.714 113.26) (width 0.25) (layer F.Cu) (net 18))
 (segment (start 128.714 113.26) (end 125.859 116.115) (width 0.25) (layer F.Cu) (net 18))
 (segment (start 125.859 116.115) (end 125.859 116.6) (width 0.25) (layer F.Cu) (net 18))
 (via (at 116.859 137.35) (size 0.6) (layers F.Cu B.Cu) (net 5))
 (via (at 128.905 126.111) (size 0.6) (layers F.Cu B.Cu) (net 10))
 (via (at 136.779 131.445) (size 0.6) (layers F.Cu B.Cu) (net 10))
 (via (at 123.571 125.349) (size 0.6) (layers F.Cu B.Cu) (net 10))
 (via (at 118.359 131.35) (size 0.6) (layers F.Cu B.Cu) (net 7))
 (via (at 121.018011 131.6) (size 0.6) (layers F.Cu B.Cu) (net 7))
 (via (at 131.699 115.189) (size 0.6) (layers F.Cu B.Cu) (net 7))
 (via (at 129.859 130.35) (size 0.6) (layers F.Cu B.Cu) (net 3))
 (via (at 129.109 131.1) (size 0.6) (layers F.Cu B.Cu) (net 4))
 (via (at 124.390696 123.513306) (size 0.6) (layers F.Cu B.Cu) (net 8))
 (via (at 123.571 124.079) (size 0.6) (layers F.Cu B.Cu) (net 9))
 (via (at 121.793 126.111) (size 0.6) (layers F.Cu B.Cu) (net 11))
 (via (at 119.327895 126.457122) (size 0.6) (layers F.Cu B.Cu) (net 12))
 (via (at 132.521259 124.437741) (size 0.6) (layers F.Cu B.Cu) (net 18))
 (via (at 125.859 116.6) (size 0.6) (layers F.Cu B.Cu) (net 18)))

